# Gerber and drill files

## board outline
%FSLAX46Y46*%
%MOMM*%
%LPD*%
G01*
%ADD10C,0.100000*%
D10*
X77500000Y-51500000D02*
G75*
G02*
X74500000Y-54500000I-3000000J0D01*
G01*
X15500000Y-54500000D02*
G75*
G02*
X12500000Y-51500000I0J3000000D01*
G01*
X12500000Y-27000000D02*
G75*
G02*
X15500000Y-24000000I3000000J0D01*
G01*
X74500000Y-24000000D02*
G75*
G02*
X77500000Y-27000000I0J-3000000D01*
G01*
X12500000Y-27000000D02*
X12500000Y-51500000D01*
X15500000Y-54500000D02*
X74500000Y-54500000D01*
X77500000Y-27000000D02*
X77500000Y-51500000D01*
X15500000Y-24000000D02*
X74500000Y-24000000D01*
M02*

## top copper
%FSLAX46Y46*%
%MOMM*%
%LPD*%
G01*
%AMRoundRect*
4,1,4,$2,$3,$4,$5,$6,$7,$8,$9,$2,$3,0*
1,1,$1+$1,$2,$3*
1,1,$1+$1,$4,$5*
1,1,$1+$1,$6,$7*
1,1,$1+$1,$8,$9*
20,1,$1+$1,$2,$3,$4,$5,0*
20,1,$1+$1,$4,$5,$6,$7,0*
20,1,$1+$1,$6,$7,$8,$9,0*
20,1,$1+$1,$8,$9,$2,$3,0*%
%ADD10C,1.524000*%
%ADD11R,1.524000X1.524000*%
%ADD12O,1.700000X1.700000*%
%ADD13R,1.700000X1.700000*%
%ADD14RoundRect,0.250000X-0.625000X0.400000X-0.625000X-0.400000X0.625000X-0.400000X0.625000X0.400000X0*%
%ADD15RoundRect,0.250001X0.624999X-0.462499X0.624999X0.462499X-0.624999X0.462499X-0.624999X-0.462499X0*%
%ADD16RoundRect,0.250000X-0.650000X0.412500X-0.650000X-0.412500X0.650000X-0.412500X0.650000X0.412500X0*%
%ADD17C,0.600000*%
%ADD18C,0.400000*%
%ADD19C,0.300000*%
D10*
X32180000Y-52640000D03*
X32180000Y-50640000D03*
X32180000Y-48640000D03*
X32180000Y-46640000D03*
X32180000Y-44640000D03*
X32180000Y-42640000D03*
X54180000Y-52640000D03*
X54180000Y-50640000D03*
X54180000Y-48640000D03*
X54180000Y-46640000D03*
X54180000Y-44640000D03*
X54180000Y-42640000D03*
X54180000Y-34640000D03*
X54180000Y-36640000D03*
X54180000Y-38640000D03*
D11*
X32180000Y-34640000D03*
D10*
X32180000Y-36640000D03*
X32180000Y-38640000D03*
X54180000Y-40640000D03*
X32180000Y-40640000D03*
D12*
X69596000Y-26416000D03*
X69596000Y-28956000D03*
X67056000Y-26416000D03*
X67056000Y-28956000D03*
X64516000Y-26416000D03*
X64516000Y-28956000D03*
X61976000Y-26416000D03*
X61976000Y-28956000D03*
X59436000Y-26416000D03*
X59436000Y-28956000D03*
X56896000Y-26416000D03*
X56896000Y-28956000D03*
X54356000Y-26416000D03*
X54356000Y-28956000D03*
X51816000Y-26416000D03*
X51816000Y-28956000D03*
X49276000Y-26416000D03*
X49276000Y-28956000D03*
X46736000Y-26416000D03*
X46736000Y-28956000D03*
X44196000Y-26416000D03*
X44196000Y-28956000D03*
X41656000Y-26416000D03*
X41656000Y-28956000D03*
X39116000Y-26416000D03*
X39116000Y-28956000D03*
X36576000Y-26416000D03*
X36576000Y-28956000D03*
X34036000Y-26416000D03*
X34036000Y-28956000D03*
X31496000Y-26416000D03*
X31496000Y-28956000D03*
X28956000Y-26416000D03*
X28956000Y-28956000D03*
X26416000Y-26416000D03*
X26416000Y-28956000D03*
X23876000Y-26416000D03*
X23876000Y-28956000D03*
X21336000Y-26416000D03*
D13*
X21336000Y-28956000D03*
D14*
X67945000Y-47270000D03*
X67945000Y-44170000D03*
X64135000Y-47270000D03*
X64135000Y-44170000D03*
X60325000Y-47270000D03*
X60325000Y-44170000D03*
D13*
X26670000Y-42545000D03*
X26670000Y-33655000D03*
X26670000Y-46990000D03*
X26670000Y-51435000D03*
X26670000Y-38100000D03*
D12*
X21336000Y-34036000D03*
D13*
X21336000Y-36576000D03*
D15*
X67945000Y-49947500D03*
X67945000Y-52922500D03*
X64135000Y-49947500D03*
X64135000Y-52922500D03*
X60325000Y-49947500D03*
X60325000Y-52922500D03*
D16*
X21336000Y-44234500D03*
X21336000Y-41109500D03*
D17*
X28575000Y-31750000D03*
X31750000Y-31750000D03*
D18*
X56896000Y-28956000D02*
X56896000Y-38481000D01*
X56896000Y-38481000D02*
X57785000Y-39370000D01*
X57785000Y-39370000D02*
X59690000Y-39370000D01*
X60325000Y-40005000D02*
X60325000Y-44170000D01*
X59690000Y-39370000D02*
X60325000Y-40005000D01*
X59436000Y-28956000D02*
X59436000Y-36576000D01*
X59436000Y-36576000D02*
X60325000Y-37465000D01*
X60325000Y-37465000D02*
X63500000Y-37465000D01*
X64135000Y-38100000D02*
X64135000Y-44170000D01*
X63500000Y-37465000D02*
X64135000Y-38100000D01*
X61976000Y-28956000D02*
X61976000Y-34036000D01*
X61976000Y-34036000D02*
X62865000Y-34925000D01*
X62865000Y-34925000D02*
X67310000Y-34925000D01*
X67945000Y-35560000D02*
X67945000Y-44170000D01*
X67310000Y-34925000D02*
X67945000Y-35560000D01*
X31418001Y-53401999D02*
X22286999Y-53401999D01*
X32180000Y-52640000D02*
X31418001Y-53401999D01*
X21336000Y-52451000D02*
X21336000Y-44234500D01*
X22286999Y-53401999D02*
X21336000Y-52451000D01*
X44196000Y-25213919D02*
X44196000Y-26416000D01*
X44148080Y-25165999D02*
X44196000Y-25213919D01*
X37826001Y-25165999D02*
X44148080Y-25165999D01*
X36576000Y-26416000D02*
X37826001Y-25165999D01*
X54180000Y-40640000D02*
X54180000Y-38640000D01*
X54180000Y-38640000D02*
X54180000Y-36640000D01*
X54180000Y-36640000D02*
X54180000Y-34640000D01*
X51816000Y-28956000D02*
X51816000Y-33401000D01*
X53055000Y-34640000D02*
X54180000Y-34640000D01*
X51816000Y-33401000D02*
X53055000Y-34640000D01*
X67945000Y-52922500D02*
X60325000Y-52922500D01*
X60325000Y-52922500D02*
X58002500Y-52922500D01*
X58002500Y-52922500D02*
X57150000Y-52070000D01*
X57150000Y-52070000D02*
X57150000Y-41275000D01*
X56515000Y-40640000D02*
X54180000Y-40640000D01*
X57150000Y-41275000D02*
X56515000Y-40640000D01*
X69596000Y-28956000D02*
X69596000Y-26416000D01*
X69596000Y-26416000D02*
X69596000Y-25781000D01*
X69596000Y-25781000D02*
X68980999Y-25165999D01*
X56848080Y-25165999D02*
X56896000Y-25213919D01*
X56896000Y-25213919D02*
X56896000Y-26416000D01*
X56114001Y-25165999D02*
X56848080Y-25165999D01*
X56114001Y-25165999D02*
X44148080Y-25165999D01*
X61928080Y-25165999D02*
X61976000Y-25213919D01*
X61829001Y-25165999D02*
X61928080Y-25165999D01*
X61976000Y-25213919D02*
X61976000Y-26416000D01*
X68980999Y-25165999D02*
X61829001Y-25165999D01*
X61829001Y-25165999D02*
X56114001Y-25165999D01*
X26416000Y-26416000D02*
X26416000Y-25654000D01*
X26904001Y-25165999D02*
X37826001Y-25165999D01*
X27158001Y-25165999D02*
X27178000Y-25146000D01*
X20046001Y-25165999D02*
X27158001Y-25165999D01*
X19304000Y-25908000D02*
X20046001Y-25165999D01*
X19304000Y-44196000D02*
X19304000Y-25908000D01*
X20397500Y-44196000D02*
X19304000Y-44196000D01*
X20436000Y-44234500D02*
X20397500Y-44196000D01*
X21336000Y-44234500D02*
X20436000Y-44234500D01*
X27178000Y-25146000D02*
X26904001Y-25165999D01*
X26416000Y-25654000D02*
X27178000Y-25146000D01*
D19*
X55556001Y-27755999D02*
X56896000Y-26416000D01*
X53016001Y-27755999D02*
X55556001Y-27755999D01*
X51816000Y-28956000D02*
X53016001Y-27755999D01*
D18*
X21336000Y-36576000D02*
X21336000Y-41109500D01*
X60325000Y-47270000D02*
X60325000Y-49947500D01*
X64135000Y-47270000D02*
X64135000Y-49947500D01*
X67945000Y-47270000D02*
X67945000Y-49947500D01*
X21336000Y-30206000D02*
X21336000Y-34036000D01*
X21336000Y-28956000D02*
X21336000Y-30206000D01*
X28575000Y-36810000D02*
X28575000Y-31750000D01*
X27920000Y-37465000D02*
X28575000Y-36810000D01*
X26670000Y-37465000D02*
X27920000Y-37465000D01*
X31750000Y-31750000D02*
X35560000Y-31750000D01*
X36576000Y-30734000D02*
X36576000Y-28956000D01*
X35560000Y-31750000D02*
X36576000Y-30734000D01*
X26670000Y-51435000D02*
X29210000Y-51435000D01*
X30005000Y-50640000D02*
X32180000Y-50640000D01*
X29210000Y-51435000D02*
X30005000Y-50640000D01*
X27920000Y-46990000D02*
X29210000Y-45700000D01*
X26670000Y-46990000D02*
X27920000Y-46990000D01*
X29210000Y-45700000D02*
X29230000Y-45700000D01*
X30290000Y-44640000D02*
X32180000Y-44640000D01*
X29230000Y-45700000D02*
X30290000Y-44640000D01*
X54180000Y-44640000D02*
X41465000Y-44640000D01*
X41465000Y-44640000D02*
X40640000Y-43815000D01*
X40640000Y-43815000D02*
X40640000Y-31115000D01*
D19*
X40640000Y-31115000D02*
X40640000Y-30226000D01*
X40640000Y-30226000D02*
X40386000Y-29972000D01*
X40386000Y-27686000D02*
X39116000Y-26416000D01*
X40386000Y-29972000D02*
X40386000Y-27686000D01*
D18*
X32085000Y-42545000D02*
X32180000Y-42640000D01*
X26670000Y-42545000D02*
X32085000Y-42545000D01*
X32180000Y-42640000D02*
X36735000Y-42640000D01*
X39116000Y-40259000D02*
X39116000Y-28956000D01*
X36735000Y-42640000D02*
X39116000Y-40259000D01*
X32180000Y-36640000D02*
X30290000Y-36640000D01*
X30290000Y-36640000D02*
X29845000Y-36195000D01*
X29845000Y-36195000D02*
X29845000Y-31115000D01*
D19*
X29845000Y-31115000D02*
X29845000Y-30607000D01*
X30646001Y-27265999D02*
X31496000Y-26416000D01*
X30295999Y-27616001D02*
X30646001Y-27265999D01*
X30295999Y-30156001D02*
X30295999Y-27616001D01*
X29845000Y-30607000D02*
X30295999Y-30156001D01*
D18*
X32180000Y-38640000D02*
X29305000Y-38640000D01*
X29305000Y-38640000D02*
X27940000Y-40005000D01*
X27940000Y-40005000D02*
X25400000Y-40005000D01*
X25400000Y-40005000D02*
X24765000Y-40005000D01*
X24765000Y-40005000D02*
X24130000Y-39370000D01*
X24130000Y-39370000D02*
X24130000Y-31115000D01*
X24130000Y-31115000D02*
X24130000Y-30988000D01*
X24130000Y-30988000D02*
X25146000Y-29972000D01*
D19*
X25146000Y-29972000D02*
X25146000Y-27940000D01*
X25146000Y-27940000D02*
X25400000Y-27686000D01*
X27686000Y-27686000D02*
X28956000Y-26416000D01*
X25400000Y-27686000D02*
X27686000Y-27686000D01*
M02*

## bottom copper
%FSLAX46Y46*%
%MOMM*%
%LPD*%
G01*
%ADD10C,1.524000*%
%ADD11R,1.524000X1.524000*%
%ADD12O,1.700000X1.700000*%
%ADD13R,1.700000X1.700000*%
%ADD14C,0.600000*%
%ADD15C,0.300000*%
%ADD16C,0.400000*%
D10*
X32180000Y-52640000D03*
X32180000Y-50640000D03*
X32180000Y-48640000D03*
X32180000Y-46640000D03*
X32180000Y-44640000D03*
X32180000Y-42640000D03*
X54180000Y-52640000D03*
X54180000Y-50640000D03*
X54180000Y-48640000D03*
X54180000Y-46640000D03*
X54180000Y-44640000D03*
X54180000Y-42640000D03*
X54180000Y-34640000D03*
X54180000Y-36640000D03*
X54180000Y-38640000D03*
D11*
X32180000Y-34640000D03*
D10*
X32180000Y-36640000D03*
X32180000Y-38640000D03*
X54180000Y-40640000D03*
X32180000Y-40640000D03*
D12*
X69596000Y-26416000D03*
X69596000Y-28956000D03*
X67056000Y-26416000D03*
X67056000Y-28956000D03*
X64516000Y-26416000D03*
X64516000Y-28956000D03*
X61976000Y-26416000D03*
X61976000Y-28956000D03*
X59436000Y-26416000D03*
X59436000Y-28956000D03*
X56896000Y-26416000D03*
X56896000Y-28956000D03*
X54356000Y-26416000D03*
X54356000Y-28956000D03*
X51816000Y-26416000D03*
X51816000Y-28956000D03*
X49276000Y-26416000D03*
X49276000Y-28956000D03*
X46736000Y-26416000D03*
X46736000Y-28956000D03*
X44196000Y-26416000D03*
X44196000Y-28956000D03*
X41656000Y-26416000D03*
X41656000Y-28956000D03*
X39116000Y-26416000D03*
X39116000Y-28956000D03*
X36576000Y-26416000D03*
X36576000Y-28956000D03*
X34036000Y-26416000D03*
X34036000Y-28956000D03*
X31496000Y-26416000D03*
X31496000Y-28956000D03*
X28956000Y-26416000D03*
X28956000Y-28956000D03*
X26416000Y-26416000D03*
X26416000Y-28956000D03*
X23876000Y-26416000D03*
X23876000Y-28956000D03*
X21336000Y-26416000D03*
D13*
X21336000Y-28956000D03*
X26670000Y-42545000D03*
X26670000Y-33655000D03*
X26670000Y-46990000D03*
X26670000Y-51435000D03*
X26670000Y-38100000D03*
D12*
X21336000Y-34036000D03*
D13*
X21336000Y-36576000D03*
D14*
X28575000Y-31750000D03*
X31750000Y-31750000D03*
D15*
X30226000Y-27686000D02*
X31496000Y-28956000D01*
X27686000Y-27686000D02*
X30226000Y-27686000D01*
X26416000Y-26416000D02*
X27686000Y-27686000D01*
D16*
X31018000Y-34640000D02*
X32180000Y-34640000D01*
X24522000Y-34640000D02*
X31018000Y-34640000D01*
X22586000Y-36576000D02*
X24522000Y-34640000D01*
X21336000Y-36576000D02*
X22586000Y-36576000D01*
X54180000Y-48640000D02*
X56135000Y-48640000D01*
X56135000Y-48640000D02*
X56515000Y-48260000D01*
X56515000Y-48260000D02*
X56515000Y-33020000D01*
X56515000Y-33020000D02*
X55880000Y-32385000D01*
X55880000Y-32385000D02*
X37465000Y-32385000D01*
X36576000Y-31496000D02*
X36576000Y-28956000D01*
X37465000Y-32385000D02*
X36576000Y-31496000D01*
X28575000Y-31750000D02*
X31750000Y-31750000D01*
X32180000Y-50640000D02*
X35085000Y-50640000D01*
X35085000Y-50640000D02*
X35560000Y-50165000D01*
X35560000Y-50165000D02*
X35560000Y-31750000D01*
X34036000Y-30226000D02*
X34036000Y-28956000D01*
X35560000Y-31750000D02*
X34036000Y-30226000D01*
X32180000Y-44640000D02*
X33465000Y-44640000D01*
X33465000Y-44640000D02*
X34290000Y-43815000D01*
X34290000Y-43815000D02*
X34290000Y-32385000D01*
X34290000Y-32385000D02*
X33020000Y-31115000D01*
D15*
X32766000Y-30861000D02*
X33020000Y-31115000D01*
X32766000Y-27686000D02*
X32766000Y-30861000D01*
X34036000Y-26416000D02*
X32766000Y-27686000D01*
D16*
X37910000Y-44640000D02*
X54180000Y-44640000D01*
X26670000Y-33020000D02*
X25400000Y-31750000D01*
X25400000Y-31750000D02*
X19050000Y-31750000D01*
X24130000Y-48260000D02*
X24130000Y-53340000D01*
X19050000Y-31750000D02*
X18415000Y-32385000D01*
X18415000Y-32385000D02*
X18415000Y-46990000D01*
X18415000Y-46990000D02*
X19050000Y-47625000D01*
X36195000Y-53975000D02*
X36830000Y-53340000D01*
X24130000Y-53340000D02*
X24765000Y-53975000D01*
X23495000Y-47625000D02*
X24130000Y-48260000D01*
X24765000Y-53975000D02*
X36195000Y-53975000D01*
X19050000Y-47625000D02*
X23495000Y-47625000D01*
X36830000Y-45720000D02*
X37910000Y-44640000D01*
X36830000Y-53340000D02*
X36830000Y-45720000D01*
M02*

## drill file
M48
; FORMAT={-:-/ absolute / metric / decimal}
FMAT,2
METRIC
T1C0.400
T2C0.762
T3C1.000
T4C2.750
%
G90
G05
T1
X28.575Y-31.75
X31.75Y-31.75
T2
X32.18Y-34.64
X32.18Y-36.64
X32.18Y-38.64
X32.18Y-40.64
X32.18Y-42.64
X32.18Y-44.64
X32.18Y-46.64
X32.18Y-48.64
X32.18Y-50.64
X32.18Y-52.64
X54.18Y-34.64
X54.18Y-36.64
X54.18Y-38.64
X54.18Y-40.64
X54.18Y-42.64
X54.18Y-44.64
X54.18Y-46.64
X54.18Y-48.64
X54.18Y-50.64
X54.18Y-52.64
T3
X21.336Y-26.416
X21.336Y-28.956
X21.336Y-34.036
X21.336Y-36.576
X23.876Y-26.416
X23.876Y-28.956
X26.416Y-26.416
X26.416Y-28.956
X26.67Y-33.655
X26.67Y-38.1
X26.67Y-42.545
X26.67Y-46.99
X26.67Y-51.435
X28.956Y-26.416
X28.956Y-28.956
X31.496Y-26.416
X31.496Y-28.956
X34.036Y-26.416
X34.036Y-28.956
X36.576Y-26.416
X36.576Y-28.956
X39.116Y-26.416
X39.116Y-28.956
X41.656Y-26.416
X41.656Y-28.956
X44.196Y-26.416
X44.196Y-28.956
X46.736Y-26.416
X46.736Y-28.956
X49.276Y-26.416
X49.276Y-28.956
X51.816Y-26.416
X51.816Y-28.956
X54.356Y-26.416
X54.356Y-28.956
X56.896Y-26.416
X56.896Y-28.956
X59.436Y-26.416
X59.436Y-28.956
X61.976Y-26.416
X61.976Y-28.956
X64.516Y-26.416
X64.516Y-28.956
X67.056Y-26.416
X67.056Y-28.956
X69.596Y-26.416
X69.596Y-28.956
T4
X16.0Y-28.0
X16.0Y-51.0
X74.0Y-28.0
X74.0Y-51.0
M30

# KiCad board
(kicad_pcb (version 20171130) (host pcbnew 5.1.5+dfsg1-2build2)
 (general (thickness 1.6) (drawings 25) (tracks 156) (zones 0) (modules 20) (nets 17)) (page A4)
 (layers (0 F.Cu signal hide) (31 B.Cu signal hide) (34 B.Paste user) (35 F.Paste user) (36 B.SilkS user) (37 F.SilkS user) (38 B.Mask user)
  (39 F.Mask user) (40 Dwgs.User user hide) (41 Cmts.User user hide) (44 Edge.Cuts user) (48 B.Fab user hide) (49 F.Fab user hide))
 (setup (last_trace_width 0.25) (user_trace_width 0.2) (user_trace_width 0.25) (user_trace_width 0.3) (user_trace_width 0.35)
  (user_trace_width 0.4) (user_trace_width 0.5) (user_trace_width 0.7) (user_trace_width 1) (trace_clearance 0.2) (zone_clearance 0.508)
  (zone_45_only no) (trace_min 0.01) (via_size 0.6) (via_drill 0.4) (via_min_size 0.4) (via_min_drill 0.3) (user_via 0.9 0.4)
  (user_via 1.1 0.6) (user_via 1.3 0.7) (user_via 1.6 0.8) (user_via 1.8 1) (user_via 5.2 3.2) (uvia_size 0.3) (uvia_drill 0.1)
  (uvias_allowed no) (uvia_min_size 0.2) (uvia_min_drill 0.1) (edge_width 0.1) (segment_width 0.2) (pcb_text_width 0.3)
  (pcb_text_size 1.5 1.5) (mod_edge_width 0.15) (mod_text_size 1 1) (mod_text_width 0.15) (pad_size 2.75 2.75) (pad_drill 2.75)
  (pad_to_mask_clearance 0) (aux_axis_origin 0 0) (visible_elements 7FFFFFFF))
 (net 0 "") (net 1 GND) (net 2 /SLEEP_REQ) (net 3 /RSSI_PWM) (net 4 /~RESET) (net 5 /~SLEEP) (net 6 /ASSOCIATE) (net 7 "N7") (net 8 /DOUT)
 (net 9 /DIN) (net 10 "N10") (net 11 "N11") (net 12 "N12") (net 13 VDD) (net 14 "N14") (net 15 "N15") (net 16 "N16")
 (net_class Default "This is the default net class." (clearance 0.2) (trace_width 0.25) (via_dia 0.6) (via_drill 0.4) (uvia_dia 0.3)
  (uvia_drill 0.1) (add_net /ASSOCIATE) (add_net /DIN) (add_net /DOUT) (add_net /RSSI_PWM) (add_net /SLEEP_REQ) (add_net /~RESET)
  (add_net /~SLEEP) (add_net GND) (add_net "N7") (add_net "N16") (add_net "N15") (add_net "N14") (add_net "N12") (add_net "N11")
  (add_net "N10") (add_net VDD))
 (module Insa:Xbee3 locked (layer F.Cu) (at 43.18 40.64)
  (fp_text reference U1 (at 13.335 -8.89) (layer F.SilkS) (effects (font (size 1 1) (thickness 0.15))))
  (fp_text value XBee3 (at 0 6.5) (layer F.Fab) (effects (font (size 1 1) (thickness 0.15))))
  (pad 10 thru_hole circle (at -11 12) (size 1.524 1.524) (drill 0.762) (layers *.Cu *.Mask) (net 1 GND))
  (pad 9 thru_hole circle (at -11 10) (size 1.524 1.524) (drill 0.762) (layers *.Cu *.Mask) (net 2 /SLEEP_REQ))
  (pad 8 thru_hole circle (at -11 8) (size 1.524 1.524) (drill 0.762) (layers *.Cu *.Mask))
  (pad 7 thru_hole circle (at -11 6) (size 1.524 1.524) (drill 0.762) (layers *.Cu *.Mask))
  (pad 6 thru_hole circle (at -11 4) (size 1.524 1.524) (drill 0.762) (layers *.Cu *.Mask) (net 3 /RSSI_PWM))
  (pad 5 thru_hole circle (at -11 2) (size 1.524 1.524) (drill 0.762) (layers *.Cu *.Mask) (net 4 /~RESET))
  (pad 11 thru_hole circle (at 11 12) (size 1.524 1.524) (drill 0.762) (layers *.Cu *.Mask))
  (pad 12 thru_hole circle (at 11 10) (size 1.524 1.524) (drill 0.762) (layers *.Cu *.Mask))
  (pad 13 thru_hole circle (at 11 8) (size 1.524 1.524) (drill 0.762) (layers *.Cu *.Mask) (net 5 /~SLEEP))
  (pad 14 thru_hole circle (at 11 6) (size 1.524 1.524) (drill 0.762) (layers *.Cu *.Mask))
  (pad 15 thru_hole circle (at 11 4) (size 1.524 1.524) (drill 0.762) (layers *.Cu *.Mask) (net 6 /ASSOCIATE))
  (pad 16 thru_hole circle (at 11 2) (size 1.524 1.524) (drill 0.762) (layers *.Cu *.Mask))
  (pad 20 thru_hole circle (at 11 -6) (size 1.524 1.524) (drill 0.762) (layers *.Cu *.Mask) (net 1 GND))
  (pad 19 thru_hole circle (at 11 -4) (size 1.524 1.524) (drill 0.762) (layers *.Cu *.Mask) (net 1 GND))
  (pad 18 thru_hole circle (at 11 -2) (size 1.524 1.524) (drill 0.762) (layers *.Cu *.Mask) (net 1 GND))
  (pad 1 thru_hole rect (at -11 -6) (size 1.524 1.524) (drill 0.762) (layers *.Cu *.Mask) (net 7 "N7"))
  (pad 2 thru_hole circle (at -11 -4) (size 1.524 1.524) (drill 0.762) (layers *.Cu *.Mask) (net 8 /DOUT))
  (pad 3 thru_hole circle (at -11 -2) (size 1.524 1.524) (drill 0.762) (layers *.Cu *.Mask) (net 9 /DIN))
  (pad 17 thru_hole circle (at 11 0) (size 1.524 1.524) (drill 0.762) (layers *.Cu *.Mask) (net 1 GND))
  (pad 4 thru_hole circle (at -11 0) (size 1.524 1.524) (drill 0.762) (layers *.Cu *.Mask)))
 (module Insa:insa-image (layer F.Cu) (at 73.66 39.37 90)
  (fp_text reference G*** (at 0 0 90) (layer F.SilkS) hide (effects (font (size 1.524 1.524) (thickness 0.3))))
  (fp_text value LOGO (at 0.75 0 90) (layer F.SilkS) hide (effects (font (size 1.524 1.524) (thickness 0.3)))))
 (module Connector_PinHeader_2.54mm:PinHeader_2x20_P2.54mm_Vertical (layer F.Cu) (at 21.336 28.956 90)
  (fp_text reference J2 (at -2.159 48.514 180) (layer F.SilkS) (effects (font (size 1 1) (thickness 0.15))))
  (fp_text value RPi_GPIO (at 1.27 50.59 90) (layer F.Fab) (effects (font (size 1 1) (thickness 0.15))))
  (pad 40 thru_hole oval (at 2.54 48.26 90) (size 1.7 1.7) (drill 1) (layers *.Cu *.Mask) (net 1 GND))
  (pad 39 thru_hole oval (at 0 48.26 90) (size 1.7 1.7) (drill 1) (layers *.Cu *.Mask) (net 1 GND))
  (pad 38 thru_hole oval (at 2.54 45.72 90) (size 1.7 1.7) (drill 1) (layers *.Cu *.Mask))
  (pad 37 thru_hole oval (at 0 45.72 90) (size 1.7 1.7) (drill 1) (layers *.Cu *.Mask))
  (pad 36 thru_hole oval (at 2.54 43.18 90) (size 1.7 1.7) (drill 1) (layers *.Cu *.Mask))
  (pad 35 thru_hole oval (at 0 43.18 90) (size 1.7 1.7) (drill 1) (layers *.Cu *.Mask))
  (pad 34 thru_hole oval (at 2.54 40.64 90) (size 1.7 1.7) (drill 1) (layers *.Cu *.Mask) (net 1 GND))
  (pad 33 thru_hole oval (at 0 40.64 90) (size 1.7 1.7) (drill 1) (layers *.Cu *.Mask) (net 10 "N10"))
  (pad 32 thru_hole oval (at 2.54 38.1 90) (size 1.7 1.7) (drill 1) (layers *.Cu *.Mask))
  (pad 31 thru_hole oval (at 0 38.1 90) (size 1.7 1.7) (drill 1) (layers *.Cu *.Mask) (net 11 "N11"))
  (pad 30 thru_hole oval (at 2.54 35.56 90) (size 1.7 1.7) (drill 1) (layers *.Cu *.Mask) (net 1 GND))
  (pad 29 thru_hole oval (at 0 35.56 90) (size 1.7 1.7) (drill 1) (layers *.Cu *.Mask) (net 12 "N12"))
  (pad 28 thru_hole oval (at 2.54 33.02 90) (size 1.7 1.7) (drill 1) (layers *.Cu *.Mask))
  (pad 27 thru_hole oval (at 0 33.02 90) (size 1.7 1.7) (drill 1) (layers *.Cu *.Mask))
  (pad 26 thru_hole oval (at 2.54 30.48 90) (size 1.7 1.7) (drill 1) (layers *.Cu *.Mask))
  (pad 25 thru_hole oval (at 0 30.48 90) (size 1.7 1.7) (drill 1) (layers *.Cu *.Mask) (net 1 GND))
  (pad 24 thru_hole oval (at 2.54 27.94 90) (size 1.7 1.7) (drill 1) (layers *.Cu *.Mask))
  (pad 23 thru_hole oval (at 0 27.94 90) (size 1.7 1.7) (drill 1) (layers *.Cu *.Mask))
  (pad 22 thru_hole oval (at 2.54 25.4 90) (size 1.7 1.7) (drill 1) (layers *.Cu *.Mask))
  (pad 21 thru_hole oval (at 0 25.4 90) (size 1.7 1.7) (drill 1) (layers *.Cu *.Mask))
  (pad 20 thru_hole oval (at 2.54 22.86 90) (size 1.7 1.7) (drill 1) (layers *.Cu *.Mask) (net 1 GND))
  (pad 19 thru_hole oval (at 0 22.86 90) (size 1.7 1.7) (drill 1) (layers *.Cu *.Mask))
  (pad 18 thru_hole oval (at 2.54 20.32 90) (size 1.7 1.7) (drill 1) (layers *.Cu *.Mask))
  (pad 17 thru_hole oval (at 0 20.32 90) (size 1.7 1.7) (drill 1) (layers *.Cu *.Mask))
  (pad 16 thru_hole oval (at 2.54 17.78 90) (size 1.7 1.7) (drill 1) (layers *.Cu *.Mask) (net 6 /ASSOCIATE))
  (pad 15 thru_hole oval (at 0 17.78 90) (size 1.7 1.7) (drill 1) (layers *.Cu *.Mask) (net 4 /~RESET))
  (pad 14 thru_hole oval (at 2.54 15.24 90) (size 1.7 1.7) (drill 1) (layers *.Cu *.Mask) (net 1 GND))
  (pad 13 thru_hole oval (at 0 15.24 90) (size 1.7 1.7) (drill 1) (layers *.Cu *.Mask) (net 5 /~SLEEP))
  (pad 12 thru_hole oval (at 2.54 12.7 90) (size 1.7 1.7) (drill 1) (layers *.Cu *.Mask) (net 3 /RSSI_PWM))
  (pad 11 thru_hole oval (at 0 12.7 90) (size 1.7 1.7) (drill 1) (layers *.Cu *.Mask) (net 2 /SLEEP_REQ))
  (pad 10 thru_hole oval (at 2.54 10.16 90) (size 1.7 1.7) (drill 1) (layers *.Cu *.Mask) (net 8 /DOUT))
  (pad 9 thru_hole oval (at 0 10.16 90) (size 1.7 1.7) (drill 1) (layers *.Cu *.Mask) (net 1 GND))
  (pad 8 thru_hole oval (at 2.54 7.62 90) (size 1.7 1.7) (drill 1) (layers *.Cu *.Mask) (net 9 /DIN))
  (pad 7 thru_hole oval (at 0 7.62 90) (size 1.7 1.7) (drill 1) (layers *.Cu *.Mask))
  (pad 6 thru_hole oval (at 2.54 5.08 90) (size 1.7 1.7) (drill 1) (layers *.Cu *.Mask) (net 1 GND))
  (pad 5 thru_hole oval (at 0 5.08 90) (size 1.7 1.7) (drill 1) (layers *.Cu *.Mask))
  (pad 4 thru_hole oval (at 2.54 2.54 90) (size 1.7 1.7) (drill 1) (layers *.Cu *.Mask))
  (pad 3 thru_hole oval (at 0 2.54 90) (size 1.7 1.7) (drill 1) (layers *.Cu *.Mask))
  (pad 2 thru_hole oval (at 2.54 0 90) (size 1.7 1.7) (drill 1) (layers *.Cu *.Mask))
  (pad 1 thru_hole rect (at 0 0 90) (size 1.7 1.7) (drill 1) (layers *.Cu *.Mask) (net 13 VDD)))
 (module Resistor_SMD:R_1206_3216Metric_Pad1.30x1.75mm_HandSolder (layer F.Cu) (at 67.945 45.72 270)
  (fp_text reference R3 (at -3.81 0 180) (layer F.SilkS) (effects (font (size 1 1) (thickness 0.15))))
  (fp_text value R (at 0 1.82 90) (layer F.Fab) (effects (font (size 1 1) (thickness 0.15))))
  (pad 2 smd roundrect (at 1.55 0 270) (size 1.3 1.75) (layers F.Cu F.Paste F.Mask) (roundrect_rratio 0.192308) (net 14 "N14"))
  (pad 1 smd roundrect (at -1.55 0 270) (size 1.3 1.75) (layers F.Cu F.Paste F.Mask) (roundrect_rratio 0.192308) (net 10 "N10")))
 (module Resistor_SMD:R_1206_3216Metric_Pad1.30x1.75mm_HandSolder (layer F.Cu) (at 64.135 45.72 270)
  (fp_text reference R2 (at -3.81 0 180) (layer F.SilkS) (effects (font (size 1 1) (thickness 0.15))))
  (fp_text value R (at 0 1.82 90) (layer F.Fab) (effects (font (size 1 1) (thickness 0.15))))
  (pad 2 smd roundrect (at 1.55 0 270) (size 1.3 1.75) (layers F.Cu F.Paste F.Mask) (roundrect_rratio 0.192308) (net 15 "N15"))
  (pad 1 smd roundrect (at -1.55 0 270) (size 1.3 1.75) (layers F.Cu F.Paste F.Mask) (roundrect_rratio 0.192308) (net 11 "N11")))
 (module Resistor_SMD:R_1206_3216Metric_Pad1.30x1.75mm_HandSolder (layer F.Cu) (at 60.325 45.72 270)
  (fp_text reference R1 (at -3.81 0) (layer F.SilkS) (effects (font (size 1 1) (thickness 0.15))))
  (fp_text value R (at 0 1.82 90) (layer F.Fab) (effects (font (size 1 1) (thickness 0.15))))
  (pad 2 smd roundrect (at 1.55 0 270) (size 1.3 1.75) (layers F.Cu F.Paste F.Mask) (roundrect_rratio 0.192308) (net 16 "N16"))
  (pad 1 smd roundrect (at -1.55 0 270) (size 1.3 1.75) (layers F.Cu F.Paste F.Mask) (roundrect_rratio 0.192308) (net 12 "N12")))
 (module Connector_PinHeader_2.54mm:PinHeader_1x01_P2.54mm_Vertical (layer F.Cu) (at 26.67 42.545 180)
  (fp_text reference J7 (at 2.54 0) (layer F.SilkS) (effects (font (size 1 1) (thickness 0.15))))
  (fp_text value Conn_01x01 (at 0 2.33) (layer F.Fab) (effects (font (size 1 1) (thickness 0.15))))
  (pad 1 thru_hole rect (at 0 0 180) (size 1.7 1.7) (drill 1) (layers *.Cu *.Mask) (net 4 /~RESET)))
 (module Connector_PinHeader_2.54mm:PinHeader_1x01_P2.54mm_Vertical (layer F.Cu) (at 26.67 33.655 180)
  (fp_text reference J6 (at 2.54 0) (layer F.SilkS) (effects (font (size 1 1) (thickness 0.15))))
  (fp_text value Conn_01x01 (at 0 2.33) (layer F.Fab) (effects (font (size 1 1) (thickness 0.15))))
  (pad 1 thru_hole rect (at 0 0 180) (size 1.7 1.7) (drill 1) (layers *.Cu *.Mask) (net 6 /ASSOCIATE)))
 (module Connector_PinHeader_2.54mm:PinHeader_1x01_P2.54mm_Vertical (layer F.Cu) (at 26.67 46.99 180)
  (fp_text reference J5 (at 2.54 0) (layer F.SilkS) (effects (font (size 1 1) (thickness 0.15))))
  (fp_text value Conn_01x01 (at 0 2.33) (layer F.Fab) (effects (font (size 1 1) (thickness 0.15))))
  (pad 1 thru_hole rect (at 0 0 180) (size 1.7 1.7) (drill 1) (layers *.Cu *.Mask) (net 3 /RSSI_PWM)))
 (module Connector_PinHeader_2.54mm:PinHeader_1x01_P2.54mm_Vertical (layer F.Cu) (at 26.67 51.435 180)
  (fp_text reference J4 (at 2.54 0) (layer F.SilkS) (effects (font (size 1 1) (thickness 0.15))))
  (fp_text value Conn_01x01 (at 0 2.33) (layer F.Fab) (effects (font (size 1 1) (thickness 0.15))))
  (pad 1 thru_hole rect (at 0 0 180) (size 1.7 1.7) (drill 1) (layers *.Cu *.Mask) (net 2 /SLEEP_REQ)))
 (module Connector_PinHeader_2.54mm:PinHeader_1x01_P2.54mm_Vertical (layer F.Cu) (at 26.67 38.1 180)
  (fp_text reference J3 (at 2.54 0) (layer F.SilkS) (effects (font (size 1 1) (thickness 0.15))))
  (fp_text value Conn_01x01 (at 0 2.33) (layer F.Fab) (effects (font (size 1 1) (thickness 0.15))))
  (pad 1 thru_hole rect (at 0 0 180) (size 1.7 1.7) (drill 1) (layers *.Cu *.Mask) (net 5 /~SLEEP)))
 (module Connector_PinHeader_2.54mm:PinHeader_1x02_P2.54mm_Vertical (layer F.Cu) (at 21.336 36.576 180)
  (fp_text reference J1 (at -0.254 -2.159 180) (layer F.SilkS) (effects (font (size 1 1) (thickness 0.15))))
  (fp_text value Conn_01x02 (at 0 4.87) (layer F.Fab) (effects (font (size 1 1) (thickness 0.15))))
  (pad 2 thru_hole oval (at 0 2.54 180) (size 1.7 1.7) (drill 1) (layers *.Cu *.Mask) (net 13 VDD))
  (pad 1 thru_hole rect (at 0 0 180) (size 1.7 1.7) (drill 1) (layers *.Cu *.Mask) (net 7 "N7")))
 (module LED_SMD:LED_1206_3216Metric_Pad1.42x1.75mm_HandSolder (layer F.Cu) (at 67.945 51.435 90)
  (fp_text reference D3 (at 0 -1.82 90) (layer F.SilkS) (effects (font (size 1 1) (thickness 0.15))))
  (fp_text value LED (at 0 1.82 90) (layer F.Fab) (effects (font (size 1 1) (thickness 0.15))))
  (pad 2 smd roundrect (at 1.4875 0 90) (size 1.425 1.75) (layers F.Cu F.Paste F.Mask) (roundrect_rratio 0.175439) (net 14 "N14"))
  (pad 1 smd roundrect (at -1.4875 0 90) (size 1.425 1.75) (layers F.Cu F.Paste F.Mask) (roundrect_rratio 0.175439) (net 1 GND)))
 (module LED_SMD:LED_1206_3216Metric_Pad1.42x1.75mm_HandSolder (layer F.Cu) (at 64.135 51.435 90)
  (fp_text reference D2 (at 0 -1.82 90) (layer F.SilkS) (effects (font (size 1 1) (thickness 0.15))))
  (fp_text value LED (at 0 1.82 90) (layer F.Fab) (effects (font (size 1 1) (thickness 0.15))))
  (pad 2 smd roundrect (at 1.4875 0 90) (size 1.425 1.75) (layers F.Cu F.Paste F.Mask) (roundrect_rratio 0.175439) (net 15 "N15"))
  (pad 1 smd roundrect (at -1.4875 0 90) (size 1.425 1.75) (layers F.Cu F.Paste F.Mask) (roundrect_rratio 0.175439) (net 1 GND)))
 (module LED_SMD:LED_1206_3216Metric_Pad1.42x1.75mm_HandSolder (layer F.Cu) (at 60.325 51.435 90)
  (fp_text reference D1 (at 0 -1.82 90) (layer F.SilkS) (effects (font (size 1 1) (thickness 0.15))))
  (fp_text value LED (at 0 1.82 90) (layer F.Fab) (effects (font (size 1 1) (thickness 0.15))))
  (pad 2 smd roundrect (at 1.4875 0 90) (size 1.425 1.75) (layers F.Cu F.Paste F.Mask) (roundrect_rratio 0.175439) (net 16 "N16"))
  (pad 1 smd roundrect (at -1.4875 0 90) (size 1.425 1.75) (layers F.Cu F.Paste F.Mask) (roundrect_rratio 0.175439) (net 1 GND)))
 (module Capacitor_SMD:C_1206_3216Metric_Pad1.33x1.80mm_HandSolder (layer F.Cu) (at 21.336 42.672 270)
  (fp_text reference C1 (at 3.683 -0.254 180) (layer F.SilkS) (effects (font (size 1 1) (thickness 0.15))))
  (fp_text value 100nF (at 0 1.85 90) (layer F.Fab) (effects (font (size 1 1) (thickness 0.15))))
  (pad 2 smd roundrect (at 1.5625 0 270) (size 1.325 1.8) (layers F.Cu F.Paste F.Mask) (roundrect_rratio 0.188679) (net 1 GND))
  (pad 1 smd roundrect (at -1.5625 0 270) (size 1.325 1.8) (layers F.Cu F.Paste F.Mask) (roundrect_rratio 0.188679) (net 7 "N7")))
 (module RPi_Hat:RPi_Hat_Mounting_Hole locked (layer F.Cu) (at 16 51)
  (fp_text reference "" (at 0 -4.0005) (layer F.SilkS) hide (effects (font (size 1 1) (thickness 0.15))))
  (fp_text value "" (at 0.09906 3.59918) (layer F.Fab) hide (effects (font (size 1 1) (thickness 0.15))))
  (pad "" np_thru_hole circle (at 0 0) (size 2.75 2.75) (drill 2.75) (layers *.Cu *.Mask) (solder_mask_margin 1.725) (clearance 1.725)))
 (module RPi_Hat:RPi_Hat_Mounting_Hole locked (layer F.Cu) (at 74 28)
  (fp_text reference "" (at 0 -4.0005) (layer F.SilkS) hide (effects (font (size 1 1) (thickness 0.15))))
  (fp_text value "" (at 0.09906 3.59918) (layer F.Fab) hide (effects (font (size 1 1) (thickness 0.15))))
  (pad "" np_thru_hole circle (at 0 0) (size 2.75 2.75) (drill 2.75) (layers *.Cu *.Mask) (solder_mask_margin 1.725) (clearance 1.725)))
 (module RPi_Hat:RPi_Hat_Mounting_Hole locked (layer F.Cu) (at 74 51)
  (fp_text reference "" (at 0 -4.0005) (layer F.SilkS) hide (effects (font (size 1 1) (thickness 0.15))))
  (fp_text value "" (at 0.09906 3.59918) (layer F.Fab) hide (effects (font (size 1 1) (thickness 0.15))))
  (pad "" np_thru_hole circle (at 0 0) (size 2.75 2.75) (drill 2.75) (layers *.Cu *.Mask) (solder_mask_margin 1.725) (clearance 1.725)))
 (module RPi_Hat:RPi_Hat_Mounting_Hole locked (layer F.Cu) (at 16 28)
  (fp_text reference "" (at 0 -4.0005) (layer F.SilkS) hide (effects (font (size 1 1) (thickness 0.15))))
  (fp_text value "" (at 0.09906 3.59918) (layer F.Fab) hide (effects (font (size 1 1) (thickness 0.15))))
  (pad "" np_thru_hole circle (at 0 0) (size 2.75 2.75) (drill 2.75) (layers *.Cu *.Mask) (solder_mask_margin 1.725) (clearance 1.725)))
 (gr_arc (start 74.5 51.5) (end 77.5 51.5) (angle 90) (layer Edge.Cuts) (width 0.1))
 (gr_arc (start 15.5 51.5) (end 15.5 54.5) (angle 90) (layer Edge.Cuts) (width 0.1))
 (gr_arc (start 15.5 27) (end 12.5 27) (angle 90) (layer Edge.Cuts) (width 0.1))
 (gr_arc (start 74.5 27) (end 74.5 24) (angle 90) (layer Edge.Cuts) (width 0.1))
 (gr_line (start 12.5 27) (end 12.5 51.5) (layer Edge.Cuts) (width 0.1))
 (gr_line (start 15.5 54.5) (end 74.5 54.5) (angle 90) (layer Edge.Cuts) (width 0.1))
 (gr_line (start 77.5 27) (end 77.5 51.5) (angle 90) (layer Edge.Cuts) (width 0.1))
 (gr_line (start 15.5 24) (end 74.5 24) (angle 90) (layer Edge.Cuts) (width 0.1))
 (segment (start 56.896 28.956) (end 56.896 38.481) (width 0.4) (layer F.Cu) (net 12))
 (segment (start 56.896 38.481) (end 57.785 39.37) (width 0.4) (layer F.Cu) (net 12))
 (segment (start 57.785 39.37) (end 59.69 39.37) (width 0.4) (layer F.Cu) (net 12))
 (segment (start 60.325 40.005) (end 60.325 44.17) (width 0.4) (layer F.Cu) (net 12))
 (segment (start 59.69 39.37) (end 60.325 40.005) (width 0.4) (layer F.Cu) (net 12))
 (segment (start 59.436 28.956) (end 59.436 36.576) (width 0.4) (layer F.Cu) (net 11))
 (segment (start 59.436 36.576) (end 60.325 37.465) (width 0.4) (layer F.Cu) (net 11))
 (segment (start 60.325 37.465) (end 63.5 37.465) (width 0.4) (layer F.Cu) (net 11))
 (segment (start 64.135 38.1) (end 64.135 44.17) (width 0.4) (layer F.Cu) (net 11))
 (segment (start 63.5 37.465) (end 64.135 38.1) (width 0.4) (layer F.Cu) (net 11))
 (segment (start 61.976 28.956) (end 61.976 34.036) (width 0.4) (layer F.Cu) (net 10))
 (segment (start 61.976 34.036) (end 62.865 34.925) (width 0.4) (layer F.Cu) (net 10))
 (segment (start 62.865 34.925) (end 67.31 34.925) (width 0.4) (layer F.Cu) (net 10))
 (segment (start 67.945 35.56) (end 67.945 44.17) (width 0.4) (layer F.Cu) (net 10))
 (segment (start 67.31 34.925) (end 67.945 35.56) (width 0.4) (layer F.Cu) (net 10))
 (segment (start 31.418001 53.401999) (end 22.286999 53.401999) (width 0.4) (layer F.Cu) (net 1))
 (segment (start 32.18 52.64) (end 31.418001 53.401999) (width 0.4) (layer F.Cu) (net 1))
 (segment (start 21.336 52.451) (end 21.336 44.2345) (width 0.4) (layer F.Cu) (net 1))
 (segment (start 22.286999 53.401999) (end 21.336 52.451) (width 0.4) (layer F.Cu) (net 1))
 (segment (start 44.196 25.213919) (end 44.196 26.416) (width 0.4) (layer F.Cu) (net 1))
 (segment (start 44.14808 25.165999) (end 44.196 25.213919) (width 0.4) (layer F.Cu) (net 1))
 (segment (start 37.826001 25.165999) (end 44.14808 25.165999) (width 0.4) (layer F.Cu) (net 1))
 (segment (start 36.576 26.416) (end 37.826001 25.165999) (width 0.4) (layer F.Cu) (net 1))
 (segment (start 54.18 40.64) (end 54.18 38.64) (width 0.4) (layer F.Cu) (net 1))
 (segment (start 54.18 38.64) (end 54.18 36.64) (width 0.4) (layer F.Cu) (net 1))
 (segment (start 54.18 36.64) (end 54.18 34.64) (width 0.4) (layer F.Cu) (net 1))
 (segment (start 51.816 28.956) (end 51.816 33.401) (width 0.4) (layer F.Cu) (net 1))
 (segment (start 53.055 34.64) (end 54.18 34.64) (width 0.4) (layer F.Cu) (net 1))
 (segment (start 51.816 33.401) (end 53.055 34.64) (width 0.4) (layer F.Cu) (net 1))
 (segment (start 67.945 52.9225) (end 60.325 52.9225) (width 0.4) (layer F.Cu) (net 1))
 (segment (start 60.325 52.9225) (end 58.0025 52.9225) (width 0.4) (layer F.Cu) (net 1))
 (segment (start 58.0025 52.9225) (end 57.15 52.07) (width 0.4) (layer F.Cu) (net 1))
 (segment (start 57.15 52.07) (end 57.15 41.275) (width 0.4) (layer F.Cu) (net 1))
 (segment (start 56.515 40.64) (end 54.18 40.64) (width 0.4) (layer F.Cu) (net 1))
 (segment (start 57.15 41.275) (end 56.515 40.64) (width 0.4) (layer F.Cu) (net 1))
 (segment (start 69.596 28.956) (end 69.596 26.416) (width 0.4) (layer F.Cu) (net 1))
 (segment (start 69.596 26.416) (end 69.596 25.781) (width 0.4) (layer F.Cu) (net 1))
 (segment (start 69.596 25.781) (end 68.980999 25.165999) (width 0.4) (layer F.Cu) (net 1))
 (segment (start 56.84808 25.165999) (end 56.896 25.213919) (width 0.4) (layer F.Cu) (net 1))
 (segment (start 56.896 25.213919) (end 56.896 26.416) (width 0.4) (layer F.Cu) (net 1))
 (segment (start 56.114001 25.165999) (end 56.84808 25.165999) (width 0.4) (layer F.Cu) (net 1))
 (segment (start 56.114001 25.165999) (end 44.14808 25.165999) (width 0.4) (layer F.Cu) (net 1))
 (segment (start 61.92808 25.165999) (end 61.976 25.213919) (width 0.4) (layer F.Cu) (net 1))
 (segment (start 61.829001 25.165999) (end 61.92808 25.165999) (width 0.4) (layer F.Cu) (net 1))
 (segment (start 61.976 25.213919) (end 61.976 26.416) (width 0.4) (layer F.Cu) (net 1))
 (segment (start 68.980999 25.165999) (end 61.829001 25.165999) (width 0.4) (layer F.Cu) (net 1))
 (segment (start 61.829001 25.165999) (end 56.114001 25.165999) (width 0.4) (layer F.Cu) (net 1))
 (segment (start 26.416 26.416) (end 26.416 25.654) (width 0.4) (layer F.Cu) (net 1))
 (segment (start 26.904001 25.165999) (end 37.826001 25.165999) (width 0.4) (layer F.Cu) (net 1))
 (segment (start 30.226 27.686) (end 31.496 28.956) (width 0.3) (layer B.Cu) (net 1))
 (segment (start 27.686 27.686) (end 30.226 27.686) (width 0.3) (layer B.Cu) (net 1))
 (segment (start 26.416 26.416) (end 27.686 27.686) (width 0.3) (layer B.Cu) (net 1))
 (segment (start 27.158001 25.165999) (end 27.178 25.146) (width 0.4) (layer F.Cu) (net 1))
 (segment (start 20.046001 25.165999) (end 27.158001 25.165999) (width 0.4) (layer F.Cu) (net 1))
 (segment (start 19.304 25.908) (end 20.046001 25.165999) (width 0.4) (layer F.Cu) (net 1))
 (segment (start 19.304 44.196) (end 19.304 25.908) (width 0.4) (layer F.Cu) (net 1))
 (segment (start 20.3975 44.196) (end 19.304 44.196) (width 0.4) (layer F.Cu) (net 1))
 (segment (start 20.436 44.2345) (end 20.3975 44.196) (width 0.4) (layer F.Cu) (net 1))
 (segment (start 21.336 44.2345) (end 20.436 44.2345) (width 0.4) (layer F.Cu) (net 1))
 (segment (start 27.178 25.146) (end 26.904001 25.165999) (width 0.4) (layer F.Cu) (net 1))
 (segment (start 26.416 25.654) (end 27.178 25.146) (width 0.4) (layer F.Cu) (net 1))
 (segment (start 55.556001 27.755999) (end 56.896 26.416) (width 0.3) (layer F.Cu) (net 1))
 (segment (start 53.016001 27.755999) (end 55.556001 27.755999) (width 0.3) (layer F.Cu) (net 1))
 (segment (start 51.816 28.956) (end 53.016001 27.755999) (width 0.3) (layer F.Cu) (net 1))
 (segment (start 21.336 36.576) (end 21.336 41.1095) (width 0.4) (layer F.Cu) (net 7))
 (segment (start 31.018 34.64) (end 32.18 34.64) (width 0.4) (layer B.Cu) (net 7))
 (segment (start 24.522 34.64) (end 31.018 34.64) (width 0.4) (layer B.Cu) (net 7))
 (segment (start 22.586 36.576) (end 24.522 34.64) (width 0.4) (layer B.Cu) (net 7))
 (segment (start 21.336 36.576) (end 22.586 36.576) (width 0.4) (layer B.Cu) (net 7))
 (segment (start 60.325 47.27) (end 60.325 49.9475) (width 0.4) (layer F.Cu) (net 16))
 (segment (start 64.135 47.27) (end 64.135 49.9475) (width 0.4) (layer F.Cu) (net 15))
 (segment (start 67.945 47.27) (end 67.945 49.9475) (width 0.4) (layer F.Cu) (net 14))
 (segment (start 21.336 30.206) (end 21.336 34.036) (width 0.4) (layer F.Cu) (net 13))
 (segment (start 21.336 28.956) (end 21.336 30.206) (width 0.4) (layer F.Cu) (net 13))
 (segment (start 54.18 48.64) (end 56.135 48.64) (width 0.4) (layer B.Cu) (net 5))
 (segment (start 56.135 48.64) (end 56.515 48.26) (width 0.4) (layer B.Cu) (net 5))
 (segment (start 56.515 48.26) (end 56.515 33.02) (width 0.4) (layer B.Cu) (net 5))
 (segment (start 56.515 33.02) (end 55.88 32.385) (width 0.4) (layer B.Cu) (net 5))
 (segment (start 55.88 32.385) (end 37.465 32.385) (width 0.4) (layer B.Cu) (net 5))
 (segment (start 36.576 31.496) (end 36.576 28.956) (width 0.4) (layer B.Cu) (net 5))
 (segment (start 37.465 32.385) (end 36.576 31.496) (width 0.4) (layer B.Cu) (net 5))
 (via (at 28.575 31.75) (size 0.6) (drill 0.4) (layers F.Cu B.Cu) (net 5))
 (segment (start 28.575 36.81) (end 28.575 31.75) (width 0.4) (layer F.Cu) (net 5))
 (segment (start 27.92 37.465) (end 28.575 36.81) (width 0.4) (layer F.Cu) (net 5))
 (segment (start 26.67 37.465) (end 27.92 37.465) (width 0.4) (layer F.Cu) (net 5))
 (via (at 31.75 31.75) (size 0.6) (drill 0.4) (layers F.Cu B.Cu) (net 5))
 (segment (start 28.575 31.75) (end 31.75 31.75) (width 0.4) (layer B.Cu) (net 5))
 (segment (start 31.75 31.75) (end 35.56 31.75) (width 0.4) (layer F.Cu) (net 5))
 (segment (start 36.576 30.734) (end 36.576 28.956) (width 0.4) (layer F.Cu) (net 5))
 (segment (start 35.56 31.75) (end 36.576 30.734) (width 0.4) (layer F.Cu) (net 5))
 (segment (start 26.67 51.435) (end 29.21 51.435) (width 0.4) (layer F.Cu) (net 2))
 (segment (start 30.005 50.64) (end 32.18 50.64) (width 0.4) (layer F.Cu) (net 2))
 (segment (start 29.21 51.435) (end 30.005 50.64) (width 0.4) (layer F.Cu) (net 2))
 (segment (start 32.18 50.64) (end 35.085 50.64) (width 0.4) (layer B.Cu) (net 2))
 (segment (start 35.085 50.64) (end 35.56 50.165) (width 0.4) (layer B.Cu) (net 2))
 (segment (start 35.56 50.165) (end 35.56 31.75) (width 0.4) (layer B.Cu) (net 2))
 (segment (start 34.036 30.226) (end 34.036 28.956) (width 0.4) (layer B.Cu) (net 2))
 (segment (start 35.56 31.75) (end 34.036 30.226) (width 0.4) (layer B.Cu) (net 2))
 (segment (start 27.92 46.99) (end 29.21 45.7) (width 0.4) (layer F.Cu) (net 3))
 (segment (start 26.67 46.99) (end 27.92 46.99) (width 0.4) (layer F.Cu) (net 3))
 (segment (start 29.21 45.7) (end 29.23 45.7) (width 0.4) (layer F.Cu) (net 3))
 (segment (start 30.29 44.64) (end 32.18 44.64) (width 0.4) (layer F.Cu) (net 3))
 (segment (start 29.23 45.7) (end 30.29 44.64) (width 0.4) (layer F.Cu) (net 3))
 (segment (start 32.18 44.64) (end 33.465 44.64) (width 0.4) (layer B.Cu) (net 3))
 (segment (start 33.465 44.64) (end 34.29 43.815) (width 0.4) (layer B.Cu) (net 3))
 (segment (start 34.29 43.815) (end 34.29 32.385) (width 0.4) (layer B.Cu) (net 3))
 (segment (start 34.29 32.385) (end 33.02 31.115) (width 0.4) (layer B.Cu) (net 3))
 (segment (start 32.766 30.861) (end 33.02 31.115) (width 0.3) (layer B.Cu) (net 3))
 (segment (start 32.766 27.686) (end 32.766 30.861) (width 0.3) (layer B.Cu) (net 3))
 (segment (start 34.036 26.416) (end 32.766 27.686) (width 0.3) (layer B.Cu) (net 3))
 (segment (start 54.18 44.64) (end 41.465 44.64) (width 0.4) (layer F.Cu) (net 6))
 (segment (start 41.465 44.64) (end 40.64 43.815) (width 0.4) (layer F.Cu) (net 6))
 (segment (start 40.64 43.815) (end 40.64 31.115) (width 0.4) (layer F.Cu) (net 6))
 (segment (start 40.64 31.115) (end 40.64 30.226) (width 0.3) (layer F.Cu) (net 6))
 (segment (start 40.64 30.226) (end 40.386 29.972) (width 0.3) (layer F.Cu) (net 6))
 (segment (start 40.386 27.686) (end 39.116 26.416) (width 0.3) (layer F.Cu) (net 6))
 (segment (start 40.386 29.972) (end 40.386 27.686) (width 0.3) (layer F.Cu) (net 6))
 (segment (start 37.91 44.64) (end 54.18 44.64) (width 0.4) (layer B.Cu) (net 6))
 (segment (start 26.67 33.02) (end 25.4 31.75) (width 0.4) (layer B.Cu) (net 6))
 (segment (start 25.4 31.75) (end 19.05 31.75) (width 0.4) (layer B.Cu) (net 6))
 (segment (start 24.13 48.26) (end 24.13 53.34) (width 0.4) (layer B.Cu) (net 6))
 (segment (start 19.05 31.75) (end 18.415 32.385) (width 0.4) (layer B.Cu) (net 6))
 (segment (start 18.415 32.385) (end 18.415 46.99) (width 0.4) (layer B.Cu) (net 6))
 (segment (start 18.415 46.99) (end 19.05 47.625) (width 0.4) (layer B.Cu) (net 6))
 (segment (start 36.195 53.975) (end 36.83 53.34) (width 0.4) (layer B.Cu) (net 6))
 (segment (start 24.13 53.34) (end 24.765 53.975) (width 0.4) (layer B.Cu) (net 6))
 (segment (start 23.495 47.625) (end 24.13 48.26) (width 0.4) (layer B.Cu) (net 6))
 (segment (start 24.765 53.975) (end 36.195 53.975) (width 0.4) (layer B.Cu) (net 6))
 (segment (start 19.05 47.625) (end 23.495 47.625) (width 0.4) (layer B.Cu) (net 6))
 (segment (start 36.83 45.72) (end 37.91 44.64) (width 0.4) (layer B.Cu) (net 6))
 (segment (start 36.83 53.34) (end 36.83 45.72) (width 0.4) (layer B.Cu) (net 6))
 (segment (start 32.085 42.545) (end 32.18 42.64) (width 0.4) (layer F.Cu) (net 4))
 (segment (start 26.67 42.545) (end 32.085 42.545) (width 0.4) (layer F.Cu) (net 4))
 (segment (start 32.18 42.64) (end 36.735 42.64) (width 0.4) (layer F.Cu) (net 4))
 (segment (start 39.116 40.259) (end 39.116 28.956) (width 0.4) (layer F.Cu) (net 4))
 (segment (start 36.735 42.64) (end 39.116 40.259) (width 0.4) (layer F.Cu) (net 4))
 (segment (start 32.18 36.64) (end 30.29 36.64) (width 0.4) (layer F.Cu) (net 8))
 (segment (start 30.29 36.64) (end 29.845 36.195) (width 0.4) (layer F.Cu) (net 8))
 (segment (start 29.845 36.195) (end 29.845 31.115) (width 0.4) (layer F.Cu) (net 8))
 (segment (start 29.845 31.115) (end 29.845 30.607) (width 0.3) (layer F.Cu) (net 8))
 (segment (start 30.646001 27.265999) (end 31.496 26.416) (width 0.3) (layer F.Cu) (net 8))
 (segment (start 30.295999 27.616001) (end 30.646001 27.265999) (width 0.3) (layer F.Cu) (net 8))
 (segment (start 30.295999 30.156001) (end 30.295999 27.616001) (width 0.3) (layer F.Cu) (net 8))
 (segment (start 29.845 30.607) (end 30.295999 30.156001) (width 0.3) (layer F.Cu) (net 8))
 (segment (start 32.18 38.64) (end 29.305 38.64) (width 0.4) (layer F.Cu) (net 9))
 (segment (start 29.305 38.64) (end 27.94 40.005) (width 0.4) (layer F.Cu) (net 9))
 (segment (start 27.94 40.005) (end 25.4 40.005) (width 0.4) (layer F.Cu) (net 9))
 (segment (start 25.4 40.005) (end 24.765 40.005) (width 0.4) (layer F.Cu) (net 9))
 (segment (start 24.765 40.005) (end 24.13 39.37) (width 0.4) (layer F.Cu) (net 9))
 (segment (start 24.13 39.37) (end 24.13 31.115) (width 0.4) (layer F.Cu) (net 9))
 (segment (start 24.13 31.115) (end 24.13 30.988) (width 0.4) (layer F.Cu) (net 9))
 (segment (start 24.13 30.988) (end 25.146 29.972) (width 0.4) (layer F.Cu) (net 9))
 (segment (start 25.146 29.972) (end 25.146 27.94) (width 0.3) (layer F.Cu) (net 9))
 (segment (start 25.146 27.94) (end 25.4 27.686) (width 0.3) (layer F.Cu) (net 9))
 (segment (start 27.686 27.686) (end 28.956 26.416) (width 0.3) (layer F.Cu) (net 9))
 (segment (start 25.4 27.686) (end 27.686 27.686) (width 0.3) (layer F.Cu) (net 9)))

